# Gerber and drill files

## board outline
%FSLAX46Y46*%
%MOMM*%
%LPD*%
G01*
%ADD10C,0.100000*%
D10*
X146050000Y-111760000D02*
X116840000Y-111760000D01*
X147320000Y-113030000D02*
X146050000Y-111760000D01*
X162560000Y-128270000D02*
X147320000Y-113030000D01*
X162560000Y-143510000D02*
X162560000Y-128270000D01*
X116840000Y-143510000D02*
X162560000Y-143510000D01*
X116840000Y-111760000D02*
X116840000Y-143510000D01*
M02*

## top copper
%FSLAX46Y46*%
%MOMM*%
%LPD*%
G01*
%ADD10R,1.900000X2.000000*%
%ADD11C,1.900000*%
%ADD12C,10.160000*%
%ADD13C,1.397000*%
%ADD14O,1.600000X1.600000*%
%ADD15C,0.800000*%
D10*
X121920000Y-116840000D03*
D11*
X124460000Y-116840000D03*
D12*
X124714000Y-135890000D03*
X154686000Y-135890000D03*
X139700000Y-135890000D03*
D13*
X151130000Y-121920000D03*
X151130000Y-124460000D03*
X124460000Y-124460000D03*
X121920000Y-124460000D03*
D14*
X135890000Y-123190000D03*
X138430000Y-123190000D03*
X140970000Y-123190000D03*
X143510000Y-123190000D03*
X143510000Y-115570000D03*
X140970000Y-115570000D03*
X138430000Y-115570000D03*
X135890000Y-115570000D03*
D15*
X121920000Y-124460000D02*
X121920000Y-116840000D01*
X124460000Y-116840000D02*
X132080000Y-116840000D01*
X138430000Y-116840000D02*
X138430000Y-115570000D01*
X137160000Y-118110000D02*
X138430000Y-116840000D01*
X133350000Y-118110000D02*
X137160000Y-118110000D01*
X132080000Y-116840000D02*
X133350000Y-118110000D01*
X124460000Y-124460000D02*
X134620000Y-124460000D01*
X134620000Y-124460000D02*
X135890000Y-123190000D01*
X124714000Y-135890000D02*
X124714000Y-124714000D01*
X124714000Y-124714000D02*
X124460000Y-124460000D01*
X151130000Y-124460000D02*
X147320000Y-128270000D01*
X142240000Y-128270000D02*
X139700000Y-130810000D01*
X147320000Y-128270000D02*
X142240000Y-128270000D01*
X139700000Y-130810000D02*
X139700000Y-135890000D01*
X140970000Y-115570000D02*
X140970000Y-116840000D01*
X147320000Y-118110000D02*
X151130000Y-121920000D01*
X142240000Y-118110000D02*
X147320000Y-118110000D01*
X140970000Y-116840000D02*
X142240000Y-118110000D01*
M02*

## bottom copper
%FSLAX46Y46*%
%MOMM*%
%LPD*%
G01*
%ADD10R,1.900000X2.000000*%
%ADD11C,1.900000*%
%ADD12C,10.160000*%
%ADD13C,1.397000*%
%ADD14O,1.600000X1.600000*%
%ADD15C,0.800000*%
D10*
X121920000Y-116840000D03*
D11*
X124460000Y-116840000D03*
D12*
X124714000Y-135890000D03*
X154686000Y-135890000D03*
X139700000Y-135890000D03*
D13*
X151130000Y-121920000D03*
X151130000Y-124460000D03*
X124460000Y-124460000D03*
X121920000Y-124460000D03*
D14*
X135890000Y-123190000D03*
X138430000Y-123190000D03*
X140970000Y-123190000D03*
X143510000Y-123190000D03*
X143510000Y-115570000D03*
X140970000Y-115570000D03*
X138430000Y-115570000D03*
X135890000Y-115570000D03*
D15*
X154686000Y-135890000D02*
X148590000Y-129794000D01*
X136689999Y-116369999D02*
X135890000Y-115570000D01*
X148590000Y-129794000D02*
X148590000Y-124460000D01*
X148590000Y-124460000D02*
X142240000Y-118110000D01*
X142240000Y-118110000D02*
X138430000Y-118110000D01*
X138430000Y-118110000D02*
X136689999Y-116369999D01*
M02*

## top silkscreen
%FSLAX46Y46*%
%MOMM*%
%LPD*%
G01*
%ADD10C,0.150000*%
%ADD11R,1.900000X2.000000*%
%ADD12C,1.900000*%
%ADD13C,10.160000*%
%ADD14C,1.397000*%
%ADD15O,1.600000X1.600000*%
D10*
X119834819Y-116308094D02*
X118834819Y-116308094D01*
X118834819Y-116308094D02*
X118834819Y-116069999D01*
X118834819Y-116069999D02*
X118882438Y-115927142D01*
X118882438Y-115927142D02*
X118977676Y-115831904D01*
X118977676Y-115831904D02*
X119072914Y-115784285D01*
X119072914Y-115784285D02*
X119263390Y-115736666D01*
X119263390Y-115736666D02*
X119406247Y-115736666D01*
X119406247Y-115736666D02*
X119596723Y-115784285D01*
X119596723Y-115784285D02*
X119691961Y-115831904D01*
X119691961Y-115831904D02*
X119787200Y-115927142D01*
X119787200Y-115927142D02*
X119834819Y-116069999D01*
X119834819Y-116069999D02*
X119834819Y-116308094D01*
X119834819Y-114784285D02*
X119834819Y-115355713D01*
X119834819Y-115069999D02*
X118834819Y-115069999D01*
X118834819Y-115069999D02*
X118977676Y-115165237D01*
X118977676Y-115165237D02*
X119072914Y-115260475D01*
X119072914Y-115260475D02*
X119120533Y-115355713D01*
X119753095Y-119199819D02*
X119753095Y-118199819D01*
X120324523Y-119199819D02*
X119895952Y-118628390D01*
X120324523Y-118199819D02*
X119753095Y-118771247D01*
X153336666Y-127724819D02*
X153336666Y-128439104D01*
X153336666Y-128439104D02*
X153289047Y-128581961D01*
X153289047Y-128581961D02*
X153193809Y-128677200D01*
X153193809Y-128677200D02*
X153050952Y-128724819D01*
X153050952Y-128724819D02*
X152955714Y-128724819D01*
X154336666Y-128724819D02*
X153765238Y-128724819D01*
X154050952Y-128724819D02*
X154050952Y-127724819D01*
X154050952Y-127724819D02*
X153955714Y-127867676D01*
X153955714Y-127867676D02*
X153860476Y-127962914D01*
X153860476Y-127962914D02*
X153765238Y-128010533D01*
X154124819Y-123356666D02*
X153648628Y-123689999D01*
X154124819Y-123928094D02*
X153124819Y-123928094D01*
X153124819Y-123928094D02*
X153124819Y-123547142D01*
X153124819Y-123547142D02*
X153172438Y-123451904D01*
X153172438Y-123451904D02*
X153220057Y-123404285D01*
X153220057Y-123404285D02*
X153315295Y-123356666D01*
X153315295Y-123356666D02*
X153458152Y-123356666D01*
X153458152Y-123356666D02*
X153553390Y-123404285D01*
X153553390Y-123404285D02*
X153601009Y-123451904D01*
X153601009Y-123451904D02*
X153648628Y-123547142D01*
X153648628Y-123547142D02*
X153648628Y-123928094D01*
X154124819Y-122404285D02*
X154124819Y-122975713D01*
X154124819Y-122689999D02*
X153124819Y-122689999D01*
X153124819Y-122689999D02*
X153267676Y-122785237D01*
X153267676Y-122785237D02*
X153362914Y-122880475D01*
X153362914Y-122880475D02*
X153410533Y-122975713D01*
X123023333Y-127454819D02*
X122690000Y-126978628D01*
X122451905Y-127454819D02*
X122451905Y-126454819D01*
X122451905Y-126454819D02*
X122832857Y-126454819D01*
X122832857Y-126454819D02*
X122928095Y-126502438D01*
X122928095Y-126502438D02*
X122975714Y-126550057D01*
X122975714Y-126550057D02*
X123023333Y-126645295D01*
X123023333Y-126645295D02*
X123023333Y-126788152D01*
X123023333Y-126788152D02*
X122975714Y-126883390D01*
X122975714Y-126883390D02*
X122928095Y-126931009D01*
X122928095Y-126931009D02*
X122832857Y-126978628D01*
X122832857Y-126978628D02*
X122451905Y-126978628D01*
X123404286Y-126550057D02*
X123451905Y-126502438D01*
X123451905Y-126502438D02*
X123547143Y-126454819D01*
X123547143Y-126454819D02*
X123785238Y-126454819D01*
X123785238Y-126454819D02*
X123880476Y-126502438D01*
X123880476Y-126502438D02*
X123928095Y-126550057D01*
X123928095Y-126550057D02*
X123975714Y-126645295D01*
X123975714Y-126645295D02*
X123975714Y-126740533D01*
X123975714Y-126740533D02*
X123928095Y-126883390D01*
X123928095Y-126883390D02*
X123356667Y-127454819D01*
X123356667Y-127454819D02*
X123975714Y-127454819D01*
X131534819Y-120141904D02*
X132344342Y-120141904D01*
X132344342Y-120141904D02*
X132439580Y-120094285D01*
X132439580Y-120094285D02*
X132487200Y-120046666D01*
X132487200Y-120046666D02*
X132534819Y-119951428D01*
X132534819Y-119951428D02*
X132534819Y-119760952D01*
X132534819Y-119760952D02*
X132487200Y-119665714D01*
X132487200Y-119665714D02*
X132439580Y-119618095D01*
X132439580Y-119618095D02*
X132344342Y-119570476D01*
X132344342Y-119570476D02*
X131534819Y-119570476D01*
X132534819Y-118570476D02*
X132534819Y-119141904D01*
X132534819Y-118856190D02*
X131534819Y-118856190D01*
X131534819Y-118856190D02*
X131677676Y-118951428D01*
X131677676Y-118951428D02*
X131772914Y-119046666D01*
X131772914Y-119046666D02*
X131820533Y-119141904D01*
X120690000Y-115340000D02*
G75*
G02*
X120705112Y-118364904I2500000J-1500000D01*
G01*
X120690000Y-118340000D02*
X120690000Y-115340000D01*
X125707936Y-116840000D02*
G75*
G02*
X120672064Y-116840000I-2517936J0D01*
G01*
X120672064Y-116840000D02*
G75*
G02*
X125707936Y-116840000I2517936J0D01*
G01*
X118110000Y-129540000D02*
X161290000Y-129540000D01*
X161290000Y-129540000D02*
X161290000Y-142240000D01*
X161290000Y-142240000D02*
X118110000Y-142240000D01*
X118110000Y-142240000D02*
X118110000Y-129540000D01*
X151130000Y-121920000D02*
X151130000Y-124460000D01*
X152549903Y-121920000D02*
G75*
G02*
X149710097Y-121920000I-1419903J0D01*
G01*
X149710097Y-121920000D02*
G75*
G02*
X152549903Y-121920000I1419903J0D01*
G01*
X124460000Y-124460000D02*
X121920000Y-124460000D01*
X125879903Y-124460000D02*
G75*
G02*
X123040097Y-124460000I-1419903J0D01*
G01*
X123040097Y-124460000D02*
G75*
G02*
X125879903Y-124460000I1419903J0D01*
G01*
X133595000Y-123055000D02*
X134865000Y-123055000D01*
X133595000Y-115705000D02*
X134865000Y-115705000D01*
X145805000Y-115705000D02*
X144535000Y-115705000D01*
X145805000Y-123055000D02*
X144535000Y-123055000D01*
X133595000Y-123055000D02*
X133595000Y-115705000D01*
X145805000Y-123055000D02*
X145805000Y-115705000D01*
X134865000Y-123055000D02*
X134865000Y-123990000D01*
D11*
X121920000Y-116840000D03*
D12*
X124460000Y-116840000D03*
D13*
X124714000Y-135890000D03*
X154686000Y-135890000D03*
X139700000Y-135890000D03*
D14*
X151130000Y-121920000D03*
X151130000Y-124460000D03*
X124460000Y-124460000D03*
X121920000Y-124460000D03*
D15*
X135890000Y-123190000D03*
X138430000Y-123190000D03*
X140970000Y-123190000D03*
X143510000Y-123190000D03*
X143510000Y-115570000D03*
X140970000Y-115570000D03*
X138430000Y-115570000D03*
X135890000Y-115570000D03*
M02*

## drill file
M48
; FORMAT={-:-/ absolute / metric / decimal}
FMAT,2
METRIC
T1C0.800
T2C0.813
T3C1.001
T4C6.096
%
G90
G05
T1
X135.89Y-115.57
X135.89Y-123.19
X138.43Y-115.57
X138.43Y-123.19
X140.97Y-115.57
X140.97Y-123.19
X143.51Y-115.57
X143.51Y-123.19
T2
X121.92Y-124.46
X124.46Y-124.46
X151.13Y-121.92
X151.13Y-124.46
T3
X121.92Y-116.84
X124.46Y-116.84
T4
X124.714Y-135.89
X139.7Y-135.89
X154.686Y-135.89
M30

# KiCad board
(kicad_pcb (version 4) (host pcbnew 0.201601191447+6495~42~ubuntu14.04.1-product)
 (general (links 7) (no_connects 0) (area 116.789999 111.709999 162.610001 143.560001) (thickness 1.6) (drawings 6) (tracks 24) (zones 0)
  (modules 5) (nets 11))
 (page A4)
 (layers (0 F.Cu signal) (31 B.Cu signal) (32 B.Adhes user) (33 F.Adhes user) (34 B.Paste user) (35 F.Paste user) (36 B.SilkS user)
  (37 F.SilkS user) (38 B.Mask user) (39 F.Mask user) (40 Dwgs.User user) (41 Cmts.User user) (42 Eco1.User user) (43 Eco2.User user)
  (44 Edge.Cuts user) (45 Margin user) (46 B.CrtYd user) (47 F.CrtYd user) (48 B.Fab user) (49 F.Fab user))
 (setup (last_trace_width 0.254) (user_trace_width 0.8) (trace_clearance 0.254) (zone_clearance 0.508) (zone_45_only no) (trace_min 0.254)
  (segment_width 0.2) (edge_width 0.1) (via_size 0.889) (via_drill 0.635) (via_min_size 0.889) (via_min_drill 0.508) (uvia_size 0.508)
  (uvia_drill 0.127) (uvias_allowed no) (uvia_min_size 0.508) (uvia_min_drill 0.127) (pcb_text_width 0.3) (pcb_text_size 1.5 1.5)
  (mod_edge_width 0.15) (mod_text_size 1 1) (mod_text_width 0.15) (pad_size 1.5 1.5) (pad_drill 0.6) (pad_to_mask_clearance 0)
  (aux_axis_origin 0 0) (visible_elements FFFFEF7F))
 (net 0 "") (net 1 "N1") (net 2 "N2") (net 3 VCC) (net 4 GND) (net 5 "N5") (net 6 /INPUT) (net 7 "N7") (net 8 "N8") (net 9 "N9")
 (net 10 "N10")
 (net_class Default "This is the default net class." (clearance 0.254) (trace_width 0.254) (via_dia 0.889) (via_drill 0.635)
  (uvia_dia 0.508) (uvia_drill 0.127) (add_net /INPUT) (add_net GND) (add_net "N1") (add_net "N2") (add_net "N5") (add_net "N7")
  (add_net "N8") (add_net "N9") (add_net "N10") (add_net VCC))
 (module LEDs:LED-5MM (layer F.Cu) (at 121.92 116.84)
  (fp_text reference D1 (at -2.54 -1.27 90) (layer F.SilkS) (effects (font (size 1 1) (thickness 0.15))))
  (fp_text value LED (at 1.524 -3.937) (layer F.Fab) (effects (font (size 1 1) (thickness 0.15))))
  (fp_arc (start 1.27 0) (end -1.23 -1.5) (angle 297.5) (layer F.SilkS) (width 0.15))
  (fp_line (start -1.23 1.5) (end -1.23 -1.5) (layer F.SilkS) (width 0.15))
  (fp_circle (center 1.27 0) (end 0.97 -2.5) (layer F.SilkS) (width 0.15))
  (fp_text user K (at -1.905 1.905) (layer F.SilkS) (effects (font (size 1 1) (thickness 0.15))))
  (pad 1 thru_hole rect (at 0 0 90) (size 2 1.9) (drill 1.00076) (layers *.Cu *.Mask F.SilkS) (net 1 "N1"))
  (pad 2 thru_hole circle (at 2.54 0) (size 1.9 1.9) (drill 1.00076) (layers *.Cu *.Mask F.SilkS) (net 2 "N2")))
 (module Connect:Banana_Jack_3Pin (layer F.Cu) (at 139.7 135.89)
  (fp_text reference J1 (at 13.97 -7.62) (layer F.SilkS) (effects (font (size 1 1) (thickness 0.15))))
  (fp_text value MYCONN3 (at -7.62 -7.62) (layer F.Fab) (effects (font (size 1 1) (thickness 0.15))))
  (fp_line (start -21.59 -6.35) (end 21.59 -6.35) (layer F.SilkS) (width 0.15))
  (fp_line (start 21.59 -6.35) (end 21.59 6.35) (layer F.SilkS) (width 0.15))
  (fp_line (start 21.59 6.35) (end -21.59 6.35) (layer F.SilkS) (width 0.15))
  (fp_line (start -21.59 6.35) (end -21.59 -6.35) (layer F.SilkS) (width 0.15))
  (pad 1 thru_hole circle (at -14.986 0) (size 10.16 10.16) (drill 6.096) (layers *.Cu *.Mask F.SilkS) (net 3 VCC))
  (pad 3 thru_hole circle (at 14.986 0) (size 10.16 10.16) (drill 6.096) (layers *.Cu *.Mask F.SilkS) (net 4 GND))
  (pad 2 thru_hole circle (at 0 0) (size 10.16 10.16) (drill 6.096) (layers *.Cu *.Mask F.SilkS) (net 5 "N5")))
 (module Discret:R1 (layer F.Cu) (at 151.13 123.19 270)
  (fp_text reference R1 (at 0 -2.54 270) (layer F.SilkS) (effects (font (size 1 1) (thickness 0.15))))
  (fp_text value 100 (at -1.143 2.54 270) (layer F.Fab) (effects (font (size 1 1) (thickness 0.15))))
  (fp_line (start -1.27 0) (end 1.27 0) (layer F.SilkS) (width 0.15))
  (fp_circle (center -1.27 0) (end -0.635 1.27) (layer F.SilkS) (width 0.15))
  (pad 1 thru_hole circle (at -1.27 0 270) (size 1.397 1.397) (drill 0.8128) (layers *.Cu *.Mask F.SilkS) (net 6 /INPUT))
  (pad 2 thru_hole circle (at 1.27 0 270) (size 1.397 1.397) (drill 0.8128) (layers *.Cu *.Mask F.SilkS) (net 5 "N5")))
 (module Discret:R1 (layer F.Cu) (at 123.19 124.46 180)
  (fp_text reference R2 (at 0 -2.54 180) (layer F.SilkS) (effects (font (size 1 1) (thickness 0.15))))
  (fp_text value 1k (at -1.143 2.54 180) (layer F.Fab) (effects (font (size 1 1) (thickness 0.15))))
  (fp_line (start -1.27 0) (end 1.27 0) (layer F.SilkS) (width 0.15))
  (fp_circle (center -1.27 0) (end -0.635 1.27) (layer F.SilkS) (width 0.15))
  (pad 1 thru_hole circle (at -1.27 0 180) (size 1.397 1.397) (drill 0.8128) (layers *.Cu *.Mask F.SilkS) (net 3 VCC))
  (pad 2 thru_hole circle (at 1.27 0 180) (size 1.397 1.397) (drill 0.8128) (layers *.Cu *.Mask F.SilkS) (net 1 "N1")))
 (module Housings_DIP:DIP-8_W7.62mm (layer F.Cu) (at 135.89 123.19 90)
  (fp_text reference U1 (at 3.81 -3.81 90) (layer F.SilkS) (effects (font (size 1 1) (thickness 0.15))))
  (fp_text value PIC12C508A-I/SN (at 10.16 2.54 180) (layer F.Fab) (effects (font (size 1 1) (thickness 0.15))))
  (fp_line (start 0.135 -2.295) (end 0.135 -1.025) (layer F.SilkS) (width 0.15))
  (fp_line (start 7.485 -2.295) (end 7.485 -1.025) (layer F.SilkS) (width 0.15))
  (fp_line (start 7.485 9.915) (end 7.485 8.645) (layer F.SilkS) (width 0.15))
  (fp_line (start 0.135 9.915) (end 0.135 8.645) (layer F.SilkS) (width 0.15))
  (fp_line (start 0.135 -2.295) (end 7.485 -2.295) (layer F.SilkS) (width 0.15))
  (fp_line (start 0.135 9.915) (end 7.485 9.915) (layer F.SilkS) (width 0.15))
  (fp_line (start 0.135 -1.025) (end -0.8 -1.025) (layer F.SilkS) (width 0.15))
  (pad 1 thru_hole oval (at 0 0 90) (size 1.6 1.6) (drill 0.8) (layers *.Cu *.Mask F.SilkS) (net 3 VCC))
  (pad 2 thru_hole oval (at 0 2.54 90) (size 1.6 1.6) (drill 0.8) (layers *.Cu *.Mask F.SilkS) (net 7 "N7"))
  (pad 3 thru_hole oval (at 0 5.08 90) (size 1.6 1.6) (drill 0.8) (layers *.Cu *.Mask F.SilkS) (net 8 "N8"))
  (pad 4 thru_hole oval (at 0 7.62 90) (size 1.6 1.6) (drill 0.8) (layers *.Cu *.Mask F.SilkS) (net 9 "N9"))
  (pad 5 thru_hole oval (at 7.62 7.62 90) (size 1.6 1.6) (drill 0.8) (layers *.Cu *.Mask F.SilkS) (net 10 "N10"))
  (pad 6 thru_hole oval (at 7.62 5.08 90) (size 1.6 1.6) (drill 0.8) (layers *.Cu *.Mask F.SilkS) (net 6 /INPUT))
  (pad 7 thru_hole oval (at 7.62 2.54 90) (size 1.6 1.6) (drill 0.8) (layers *.Cu *.Mask F.SilkS) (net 2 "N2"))
  (pad 8 thru_hole oval (at 7.62 0 90) (size 1.6 1.6) (drill 0.8) (layers *.Cu *.Mask F.SilkS) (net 4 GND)))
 (gr_line (start 146.05 111.76) (end 116.84 111.76) (angle 90) (layer Edge.Cuts) (width 0.1))
 (gr_line (start 147.32 113.03) (end 146.05 111.76) (angle 90) (layer Edge.Cuts) (width 0.1))
 (gr_line (start 162.56 128.27) (end 147.32 113.03) (angle 90) (layer Edge.Cuts) (width 0.1))
 (gr_line (start 162.56 143.51) (end 162.56 128.27) (angle 90) (layer Edge.Cuts) (width 0.1))
 (gr_line (start 116.84 143.51) (end 162.56 143.51) (angle 90) (layer Edge.Cuts) (width 0.1))
 (gr_line (start 116.84 111.76) (end 116.84 143.51) (angle 90) (layer Edge.Cuts) (width 0.1))
 (segment (start 121.92 124.46) (end 121.92 116.84) (width 0.8) (layer F.Cu) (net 1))
 (segment (start 124.46 116.84) (end 132.08 116.84) (width 0.8) (layer F.Cu) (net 2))
 (segment (start 138.43 116.84) (end 138.43 115.57) (width 0.8) (layer F.Cu) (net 2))
 (segment (start 137.16 118.11) (end 138.43 116.84) (width 0.8) (layer F.Cu) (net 2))
 (segment (start 133.35 118.11) (end 137.16 118.11) (width 0.8) (layer F.Cu) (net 2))
 (segment (start 132.08 116.84) (end 133.35 118.11) (width 0.8) (layer F.Cu) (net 2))
 (segment (start 124.46 124.46) (end 134.62 124.46) (width 0.8) (layer F.Cu) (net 3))
 (segment (start 134.62 124.46) (end 135.89 123.19) (width 0.8) (layer F.Cu) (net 3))
 (segment (start 124.714 135.89) (end 124.714 124.714) (width 0.8) (layer F.Cu) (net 3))
 (segment (start 124.714 124.714) (end 124.46 124.46) (width 0.8) (layer F.Cu) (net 3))
 (segment (start 154.686 135.89) (end 148.59 129.794) (width 0.8) (layer B.Cu) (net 4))
 (segment (start 136.689999 116.369999) (end 135.89 115.57) (width 0.8) (layer B.Cu) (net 4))
 (segment (start 148.59 129.794) (end 148.59 124.46) (width 0.8) (layer B.Cu) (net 4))
 (segment (start 148.59 124.46) (end 142.24 118.11) (width 0.8) (layer B.Cu) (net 4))
 (segment (start 142.24 118.11) (end 138.43 118.11) (width 0.8) (layer B.Cu) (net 4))
 (segment (start 138.43 118.11) (end 136.689999 116.369999) (width 0.8) (layer B.Cu) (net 4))
 (segment (start 151.13 124.46) (end 147.32 128.27) (width 0.8) (layer F.Cu) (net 5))
 (segment (start 142.24 128.27) (end 139.7 130.81) (width 0.8) (layer F.Cu) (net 5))
 (segment (start 147.32 128.27) (end 142.24 128.27) (width 0.8) (layer F.Cu) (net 5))
 (segment (start 139.7 130.81) (end 139.7 135.89) (width 0.8) (layer F.Cu) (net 5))
 (segment (start 140.97 115.57) (end 140.97 116.84) (width 0.8) (layer F.Cu) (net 6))
 (segment (start 147.32 118.11) (end 151.13 121.92) (width 0.8) (layer F.Cu) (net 6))
 (segment (start 142.24 118.11) (end 147.32 118.11) (width 0.8) (layer F.Cu) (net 6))
 (segment (start 140.97 116.84) (end 142.24 118.11) (width 0.8) (layer F.Cu) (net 6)))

